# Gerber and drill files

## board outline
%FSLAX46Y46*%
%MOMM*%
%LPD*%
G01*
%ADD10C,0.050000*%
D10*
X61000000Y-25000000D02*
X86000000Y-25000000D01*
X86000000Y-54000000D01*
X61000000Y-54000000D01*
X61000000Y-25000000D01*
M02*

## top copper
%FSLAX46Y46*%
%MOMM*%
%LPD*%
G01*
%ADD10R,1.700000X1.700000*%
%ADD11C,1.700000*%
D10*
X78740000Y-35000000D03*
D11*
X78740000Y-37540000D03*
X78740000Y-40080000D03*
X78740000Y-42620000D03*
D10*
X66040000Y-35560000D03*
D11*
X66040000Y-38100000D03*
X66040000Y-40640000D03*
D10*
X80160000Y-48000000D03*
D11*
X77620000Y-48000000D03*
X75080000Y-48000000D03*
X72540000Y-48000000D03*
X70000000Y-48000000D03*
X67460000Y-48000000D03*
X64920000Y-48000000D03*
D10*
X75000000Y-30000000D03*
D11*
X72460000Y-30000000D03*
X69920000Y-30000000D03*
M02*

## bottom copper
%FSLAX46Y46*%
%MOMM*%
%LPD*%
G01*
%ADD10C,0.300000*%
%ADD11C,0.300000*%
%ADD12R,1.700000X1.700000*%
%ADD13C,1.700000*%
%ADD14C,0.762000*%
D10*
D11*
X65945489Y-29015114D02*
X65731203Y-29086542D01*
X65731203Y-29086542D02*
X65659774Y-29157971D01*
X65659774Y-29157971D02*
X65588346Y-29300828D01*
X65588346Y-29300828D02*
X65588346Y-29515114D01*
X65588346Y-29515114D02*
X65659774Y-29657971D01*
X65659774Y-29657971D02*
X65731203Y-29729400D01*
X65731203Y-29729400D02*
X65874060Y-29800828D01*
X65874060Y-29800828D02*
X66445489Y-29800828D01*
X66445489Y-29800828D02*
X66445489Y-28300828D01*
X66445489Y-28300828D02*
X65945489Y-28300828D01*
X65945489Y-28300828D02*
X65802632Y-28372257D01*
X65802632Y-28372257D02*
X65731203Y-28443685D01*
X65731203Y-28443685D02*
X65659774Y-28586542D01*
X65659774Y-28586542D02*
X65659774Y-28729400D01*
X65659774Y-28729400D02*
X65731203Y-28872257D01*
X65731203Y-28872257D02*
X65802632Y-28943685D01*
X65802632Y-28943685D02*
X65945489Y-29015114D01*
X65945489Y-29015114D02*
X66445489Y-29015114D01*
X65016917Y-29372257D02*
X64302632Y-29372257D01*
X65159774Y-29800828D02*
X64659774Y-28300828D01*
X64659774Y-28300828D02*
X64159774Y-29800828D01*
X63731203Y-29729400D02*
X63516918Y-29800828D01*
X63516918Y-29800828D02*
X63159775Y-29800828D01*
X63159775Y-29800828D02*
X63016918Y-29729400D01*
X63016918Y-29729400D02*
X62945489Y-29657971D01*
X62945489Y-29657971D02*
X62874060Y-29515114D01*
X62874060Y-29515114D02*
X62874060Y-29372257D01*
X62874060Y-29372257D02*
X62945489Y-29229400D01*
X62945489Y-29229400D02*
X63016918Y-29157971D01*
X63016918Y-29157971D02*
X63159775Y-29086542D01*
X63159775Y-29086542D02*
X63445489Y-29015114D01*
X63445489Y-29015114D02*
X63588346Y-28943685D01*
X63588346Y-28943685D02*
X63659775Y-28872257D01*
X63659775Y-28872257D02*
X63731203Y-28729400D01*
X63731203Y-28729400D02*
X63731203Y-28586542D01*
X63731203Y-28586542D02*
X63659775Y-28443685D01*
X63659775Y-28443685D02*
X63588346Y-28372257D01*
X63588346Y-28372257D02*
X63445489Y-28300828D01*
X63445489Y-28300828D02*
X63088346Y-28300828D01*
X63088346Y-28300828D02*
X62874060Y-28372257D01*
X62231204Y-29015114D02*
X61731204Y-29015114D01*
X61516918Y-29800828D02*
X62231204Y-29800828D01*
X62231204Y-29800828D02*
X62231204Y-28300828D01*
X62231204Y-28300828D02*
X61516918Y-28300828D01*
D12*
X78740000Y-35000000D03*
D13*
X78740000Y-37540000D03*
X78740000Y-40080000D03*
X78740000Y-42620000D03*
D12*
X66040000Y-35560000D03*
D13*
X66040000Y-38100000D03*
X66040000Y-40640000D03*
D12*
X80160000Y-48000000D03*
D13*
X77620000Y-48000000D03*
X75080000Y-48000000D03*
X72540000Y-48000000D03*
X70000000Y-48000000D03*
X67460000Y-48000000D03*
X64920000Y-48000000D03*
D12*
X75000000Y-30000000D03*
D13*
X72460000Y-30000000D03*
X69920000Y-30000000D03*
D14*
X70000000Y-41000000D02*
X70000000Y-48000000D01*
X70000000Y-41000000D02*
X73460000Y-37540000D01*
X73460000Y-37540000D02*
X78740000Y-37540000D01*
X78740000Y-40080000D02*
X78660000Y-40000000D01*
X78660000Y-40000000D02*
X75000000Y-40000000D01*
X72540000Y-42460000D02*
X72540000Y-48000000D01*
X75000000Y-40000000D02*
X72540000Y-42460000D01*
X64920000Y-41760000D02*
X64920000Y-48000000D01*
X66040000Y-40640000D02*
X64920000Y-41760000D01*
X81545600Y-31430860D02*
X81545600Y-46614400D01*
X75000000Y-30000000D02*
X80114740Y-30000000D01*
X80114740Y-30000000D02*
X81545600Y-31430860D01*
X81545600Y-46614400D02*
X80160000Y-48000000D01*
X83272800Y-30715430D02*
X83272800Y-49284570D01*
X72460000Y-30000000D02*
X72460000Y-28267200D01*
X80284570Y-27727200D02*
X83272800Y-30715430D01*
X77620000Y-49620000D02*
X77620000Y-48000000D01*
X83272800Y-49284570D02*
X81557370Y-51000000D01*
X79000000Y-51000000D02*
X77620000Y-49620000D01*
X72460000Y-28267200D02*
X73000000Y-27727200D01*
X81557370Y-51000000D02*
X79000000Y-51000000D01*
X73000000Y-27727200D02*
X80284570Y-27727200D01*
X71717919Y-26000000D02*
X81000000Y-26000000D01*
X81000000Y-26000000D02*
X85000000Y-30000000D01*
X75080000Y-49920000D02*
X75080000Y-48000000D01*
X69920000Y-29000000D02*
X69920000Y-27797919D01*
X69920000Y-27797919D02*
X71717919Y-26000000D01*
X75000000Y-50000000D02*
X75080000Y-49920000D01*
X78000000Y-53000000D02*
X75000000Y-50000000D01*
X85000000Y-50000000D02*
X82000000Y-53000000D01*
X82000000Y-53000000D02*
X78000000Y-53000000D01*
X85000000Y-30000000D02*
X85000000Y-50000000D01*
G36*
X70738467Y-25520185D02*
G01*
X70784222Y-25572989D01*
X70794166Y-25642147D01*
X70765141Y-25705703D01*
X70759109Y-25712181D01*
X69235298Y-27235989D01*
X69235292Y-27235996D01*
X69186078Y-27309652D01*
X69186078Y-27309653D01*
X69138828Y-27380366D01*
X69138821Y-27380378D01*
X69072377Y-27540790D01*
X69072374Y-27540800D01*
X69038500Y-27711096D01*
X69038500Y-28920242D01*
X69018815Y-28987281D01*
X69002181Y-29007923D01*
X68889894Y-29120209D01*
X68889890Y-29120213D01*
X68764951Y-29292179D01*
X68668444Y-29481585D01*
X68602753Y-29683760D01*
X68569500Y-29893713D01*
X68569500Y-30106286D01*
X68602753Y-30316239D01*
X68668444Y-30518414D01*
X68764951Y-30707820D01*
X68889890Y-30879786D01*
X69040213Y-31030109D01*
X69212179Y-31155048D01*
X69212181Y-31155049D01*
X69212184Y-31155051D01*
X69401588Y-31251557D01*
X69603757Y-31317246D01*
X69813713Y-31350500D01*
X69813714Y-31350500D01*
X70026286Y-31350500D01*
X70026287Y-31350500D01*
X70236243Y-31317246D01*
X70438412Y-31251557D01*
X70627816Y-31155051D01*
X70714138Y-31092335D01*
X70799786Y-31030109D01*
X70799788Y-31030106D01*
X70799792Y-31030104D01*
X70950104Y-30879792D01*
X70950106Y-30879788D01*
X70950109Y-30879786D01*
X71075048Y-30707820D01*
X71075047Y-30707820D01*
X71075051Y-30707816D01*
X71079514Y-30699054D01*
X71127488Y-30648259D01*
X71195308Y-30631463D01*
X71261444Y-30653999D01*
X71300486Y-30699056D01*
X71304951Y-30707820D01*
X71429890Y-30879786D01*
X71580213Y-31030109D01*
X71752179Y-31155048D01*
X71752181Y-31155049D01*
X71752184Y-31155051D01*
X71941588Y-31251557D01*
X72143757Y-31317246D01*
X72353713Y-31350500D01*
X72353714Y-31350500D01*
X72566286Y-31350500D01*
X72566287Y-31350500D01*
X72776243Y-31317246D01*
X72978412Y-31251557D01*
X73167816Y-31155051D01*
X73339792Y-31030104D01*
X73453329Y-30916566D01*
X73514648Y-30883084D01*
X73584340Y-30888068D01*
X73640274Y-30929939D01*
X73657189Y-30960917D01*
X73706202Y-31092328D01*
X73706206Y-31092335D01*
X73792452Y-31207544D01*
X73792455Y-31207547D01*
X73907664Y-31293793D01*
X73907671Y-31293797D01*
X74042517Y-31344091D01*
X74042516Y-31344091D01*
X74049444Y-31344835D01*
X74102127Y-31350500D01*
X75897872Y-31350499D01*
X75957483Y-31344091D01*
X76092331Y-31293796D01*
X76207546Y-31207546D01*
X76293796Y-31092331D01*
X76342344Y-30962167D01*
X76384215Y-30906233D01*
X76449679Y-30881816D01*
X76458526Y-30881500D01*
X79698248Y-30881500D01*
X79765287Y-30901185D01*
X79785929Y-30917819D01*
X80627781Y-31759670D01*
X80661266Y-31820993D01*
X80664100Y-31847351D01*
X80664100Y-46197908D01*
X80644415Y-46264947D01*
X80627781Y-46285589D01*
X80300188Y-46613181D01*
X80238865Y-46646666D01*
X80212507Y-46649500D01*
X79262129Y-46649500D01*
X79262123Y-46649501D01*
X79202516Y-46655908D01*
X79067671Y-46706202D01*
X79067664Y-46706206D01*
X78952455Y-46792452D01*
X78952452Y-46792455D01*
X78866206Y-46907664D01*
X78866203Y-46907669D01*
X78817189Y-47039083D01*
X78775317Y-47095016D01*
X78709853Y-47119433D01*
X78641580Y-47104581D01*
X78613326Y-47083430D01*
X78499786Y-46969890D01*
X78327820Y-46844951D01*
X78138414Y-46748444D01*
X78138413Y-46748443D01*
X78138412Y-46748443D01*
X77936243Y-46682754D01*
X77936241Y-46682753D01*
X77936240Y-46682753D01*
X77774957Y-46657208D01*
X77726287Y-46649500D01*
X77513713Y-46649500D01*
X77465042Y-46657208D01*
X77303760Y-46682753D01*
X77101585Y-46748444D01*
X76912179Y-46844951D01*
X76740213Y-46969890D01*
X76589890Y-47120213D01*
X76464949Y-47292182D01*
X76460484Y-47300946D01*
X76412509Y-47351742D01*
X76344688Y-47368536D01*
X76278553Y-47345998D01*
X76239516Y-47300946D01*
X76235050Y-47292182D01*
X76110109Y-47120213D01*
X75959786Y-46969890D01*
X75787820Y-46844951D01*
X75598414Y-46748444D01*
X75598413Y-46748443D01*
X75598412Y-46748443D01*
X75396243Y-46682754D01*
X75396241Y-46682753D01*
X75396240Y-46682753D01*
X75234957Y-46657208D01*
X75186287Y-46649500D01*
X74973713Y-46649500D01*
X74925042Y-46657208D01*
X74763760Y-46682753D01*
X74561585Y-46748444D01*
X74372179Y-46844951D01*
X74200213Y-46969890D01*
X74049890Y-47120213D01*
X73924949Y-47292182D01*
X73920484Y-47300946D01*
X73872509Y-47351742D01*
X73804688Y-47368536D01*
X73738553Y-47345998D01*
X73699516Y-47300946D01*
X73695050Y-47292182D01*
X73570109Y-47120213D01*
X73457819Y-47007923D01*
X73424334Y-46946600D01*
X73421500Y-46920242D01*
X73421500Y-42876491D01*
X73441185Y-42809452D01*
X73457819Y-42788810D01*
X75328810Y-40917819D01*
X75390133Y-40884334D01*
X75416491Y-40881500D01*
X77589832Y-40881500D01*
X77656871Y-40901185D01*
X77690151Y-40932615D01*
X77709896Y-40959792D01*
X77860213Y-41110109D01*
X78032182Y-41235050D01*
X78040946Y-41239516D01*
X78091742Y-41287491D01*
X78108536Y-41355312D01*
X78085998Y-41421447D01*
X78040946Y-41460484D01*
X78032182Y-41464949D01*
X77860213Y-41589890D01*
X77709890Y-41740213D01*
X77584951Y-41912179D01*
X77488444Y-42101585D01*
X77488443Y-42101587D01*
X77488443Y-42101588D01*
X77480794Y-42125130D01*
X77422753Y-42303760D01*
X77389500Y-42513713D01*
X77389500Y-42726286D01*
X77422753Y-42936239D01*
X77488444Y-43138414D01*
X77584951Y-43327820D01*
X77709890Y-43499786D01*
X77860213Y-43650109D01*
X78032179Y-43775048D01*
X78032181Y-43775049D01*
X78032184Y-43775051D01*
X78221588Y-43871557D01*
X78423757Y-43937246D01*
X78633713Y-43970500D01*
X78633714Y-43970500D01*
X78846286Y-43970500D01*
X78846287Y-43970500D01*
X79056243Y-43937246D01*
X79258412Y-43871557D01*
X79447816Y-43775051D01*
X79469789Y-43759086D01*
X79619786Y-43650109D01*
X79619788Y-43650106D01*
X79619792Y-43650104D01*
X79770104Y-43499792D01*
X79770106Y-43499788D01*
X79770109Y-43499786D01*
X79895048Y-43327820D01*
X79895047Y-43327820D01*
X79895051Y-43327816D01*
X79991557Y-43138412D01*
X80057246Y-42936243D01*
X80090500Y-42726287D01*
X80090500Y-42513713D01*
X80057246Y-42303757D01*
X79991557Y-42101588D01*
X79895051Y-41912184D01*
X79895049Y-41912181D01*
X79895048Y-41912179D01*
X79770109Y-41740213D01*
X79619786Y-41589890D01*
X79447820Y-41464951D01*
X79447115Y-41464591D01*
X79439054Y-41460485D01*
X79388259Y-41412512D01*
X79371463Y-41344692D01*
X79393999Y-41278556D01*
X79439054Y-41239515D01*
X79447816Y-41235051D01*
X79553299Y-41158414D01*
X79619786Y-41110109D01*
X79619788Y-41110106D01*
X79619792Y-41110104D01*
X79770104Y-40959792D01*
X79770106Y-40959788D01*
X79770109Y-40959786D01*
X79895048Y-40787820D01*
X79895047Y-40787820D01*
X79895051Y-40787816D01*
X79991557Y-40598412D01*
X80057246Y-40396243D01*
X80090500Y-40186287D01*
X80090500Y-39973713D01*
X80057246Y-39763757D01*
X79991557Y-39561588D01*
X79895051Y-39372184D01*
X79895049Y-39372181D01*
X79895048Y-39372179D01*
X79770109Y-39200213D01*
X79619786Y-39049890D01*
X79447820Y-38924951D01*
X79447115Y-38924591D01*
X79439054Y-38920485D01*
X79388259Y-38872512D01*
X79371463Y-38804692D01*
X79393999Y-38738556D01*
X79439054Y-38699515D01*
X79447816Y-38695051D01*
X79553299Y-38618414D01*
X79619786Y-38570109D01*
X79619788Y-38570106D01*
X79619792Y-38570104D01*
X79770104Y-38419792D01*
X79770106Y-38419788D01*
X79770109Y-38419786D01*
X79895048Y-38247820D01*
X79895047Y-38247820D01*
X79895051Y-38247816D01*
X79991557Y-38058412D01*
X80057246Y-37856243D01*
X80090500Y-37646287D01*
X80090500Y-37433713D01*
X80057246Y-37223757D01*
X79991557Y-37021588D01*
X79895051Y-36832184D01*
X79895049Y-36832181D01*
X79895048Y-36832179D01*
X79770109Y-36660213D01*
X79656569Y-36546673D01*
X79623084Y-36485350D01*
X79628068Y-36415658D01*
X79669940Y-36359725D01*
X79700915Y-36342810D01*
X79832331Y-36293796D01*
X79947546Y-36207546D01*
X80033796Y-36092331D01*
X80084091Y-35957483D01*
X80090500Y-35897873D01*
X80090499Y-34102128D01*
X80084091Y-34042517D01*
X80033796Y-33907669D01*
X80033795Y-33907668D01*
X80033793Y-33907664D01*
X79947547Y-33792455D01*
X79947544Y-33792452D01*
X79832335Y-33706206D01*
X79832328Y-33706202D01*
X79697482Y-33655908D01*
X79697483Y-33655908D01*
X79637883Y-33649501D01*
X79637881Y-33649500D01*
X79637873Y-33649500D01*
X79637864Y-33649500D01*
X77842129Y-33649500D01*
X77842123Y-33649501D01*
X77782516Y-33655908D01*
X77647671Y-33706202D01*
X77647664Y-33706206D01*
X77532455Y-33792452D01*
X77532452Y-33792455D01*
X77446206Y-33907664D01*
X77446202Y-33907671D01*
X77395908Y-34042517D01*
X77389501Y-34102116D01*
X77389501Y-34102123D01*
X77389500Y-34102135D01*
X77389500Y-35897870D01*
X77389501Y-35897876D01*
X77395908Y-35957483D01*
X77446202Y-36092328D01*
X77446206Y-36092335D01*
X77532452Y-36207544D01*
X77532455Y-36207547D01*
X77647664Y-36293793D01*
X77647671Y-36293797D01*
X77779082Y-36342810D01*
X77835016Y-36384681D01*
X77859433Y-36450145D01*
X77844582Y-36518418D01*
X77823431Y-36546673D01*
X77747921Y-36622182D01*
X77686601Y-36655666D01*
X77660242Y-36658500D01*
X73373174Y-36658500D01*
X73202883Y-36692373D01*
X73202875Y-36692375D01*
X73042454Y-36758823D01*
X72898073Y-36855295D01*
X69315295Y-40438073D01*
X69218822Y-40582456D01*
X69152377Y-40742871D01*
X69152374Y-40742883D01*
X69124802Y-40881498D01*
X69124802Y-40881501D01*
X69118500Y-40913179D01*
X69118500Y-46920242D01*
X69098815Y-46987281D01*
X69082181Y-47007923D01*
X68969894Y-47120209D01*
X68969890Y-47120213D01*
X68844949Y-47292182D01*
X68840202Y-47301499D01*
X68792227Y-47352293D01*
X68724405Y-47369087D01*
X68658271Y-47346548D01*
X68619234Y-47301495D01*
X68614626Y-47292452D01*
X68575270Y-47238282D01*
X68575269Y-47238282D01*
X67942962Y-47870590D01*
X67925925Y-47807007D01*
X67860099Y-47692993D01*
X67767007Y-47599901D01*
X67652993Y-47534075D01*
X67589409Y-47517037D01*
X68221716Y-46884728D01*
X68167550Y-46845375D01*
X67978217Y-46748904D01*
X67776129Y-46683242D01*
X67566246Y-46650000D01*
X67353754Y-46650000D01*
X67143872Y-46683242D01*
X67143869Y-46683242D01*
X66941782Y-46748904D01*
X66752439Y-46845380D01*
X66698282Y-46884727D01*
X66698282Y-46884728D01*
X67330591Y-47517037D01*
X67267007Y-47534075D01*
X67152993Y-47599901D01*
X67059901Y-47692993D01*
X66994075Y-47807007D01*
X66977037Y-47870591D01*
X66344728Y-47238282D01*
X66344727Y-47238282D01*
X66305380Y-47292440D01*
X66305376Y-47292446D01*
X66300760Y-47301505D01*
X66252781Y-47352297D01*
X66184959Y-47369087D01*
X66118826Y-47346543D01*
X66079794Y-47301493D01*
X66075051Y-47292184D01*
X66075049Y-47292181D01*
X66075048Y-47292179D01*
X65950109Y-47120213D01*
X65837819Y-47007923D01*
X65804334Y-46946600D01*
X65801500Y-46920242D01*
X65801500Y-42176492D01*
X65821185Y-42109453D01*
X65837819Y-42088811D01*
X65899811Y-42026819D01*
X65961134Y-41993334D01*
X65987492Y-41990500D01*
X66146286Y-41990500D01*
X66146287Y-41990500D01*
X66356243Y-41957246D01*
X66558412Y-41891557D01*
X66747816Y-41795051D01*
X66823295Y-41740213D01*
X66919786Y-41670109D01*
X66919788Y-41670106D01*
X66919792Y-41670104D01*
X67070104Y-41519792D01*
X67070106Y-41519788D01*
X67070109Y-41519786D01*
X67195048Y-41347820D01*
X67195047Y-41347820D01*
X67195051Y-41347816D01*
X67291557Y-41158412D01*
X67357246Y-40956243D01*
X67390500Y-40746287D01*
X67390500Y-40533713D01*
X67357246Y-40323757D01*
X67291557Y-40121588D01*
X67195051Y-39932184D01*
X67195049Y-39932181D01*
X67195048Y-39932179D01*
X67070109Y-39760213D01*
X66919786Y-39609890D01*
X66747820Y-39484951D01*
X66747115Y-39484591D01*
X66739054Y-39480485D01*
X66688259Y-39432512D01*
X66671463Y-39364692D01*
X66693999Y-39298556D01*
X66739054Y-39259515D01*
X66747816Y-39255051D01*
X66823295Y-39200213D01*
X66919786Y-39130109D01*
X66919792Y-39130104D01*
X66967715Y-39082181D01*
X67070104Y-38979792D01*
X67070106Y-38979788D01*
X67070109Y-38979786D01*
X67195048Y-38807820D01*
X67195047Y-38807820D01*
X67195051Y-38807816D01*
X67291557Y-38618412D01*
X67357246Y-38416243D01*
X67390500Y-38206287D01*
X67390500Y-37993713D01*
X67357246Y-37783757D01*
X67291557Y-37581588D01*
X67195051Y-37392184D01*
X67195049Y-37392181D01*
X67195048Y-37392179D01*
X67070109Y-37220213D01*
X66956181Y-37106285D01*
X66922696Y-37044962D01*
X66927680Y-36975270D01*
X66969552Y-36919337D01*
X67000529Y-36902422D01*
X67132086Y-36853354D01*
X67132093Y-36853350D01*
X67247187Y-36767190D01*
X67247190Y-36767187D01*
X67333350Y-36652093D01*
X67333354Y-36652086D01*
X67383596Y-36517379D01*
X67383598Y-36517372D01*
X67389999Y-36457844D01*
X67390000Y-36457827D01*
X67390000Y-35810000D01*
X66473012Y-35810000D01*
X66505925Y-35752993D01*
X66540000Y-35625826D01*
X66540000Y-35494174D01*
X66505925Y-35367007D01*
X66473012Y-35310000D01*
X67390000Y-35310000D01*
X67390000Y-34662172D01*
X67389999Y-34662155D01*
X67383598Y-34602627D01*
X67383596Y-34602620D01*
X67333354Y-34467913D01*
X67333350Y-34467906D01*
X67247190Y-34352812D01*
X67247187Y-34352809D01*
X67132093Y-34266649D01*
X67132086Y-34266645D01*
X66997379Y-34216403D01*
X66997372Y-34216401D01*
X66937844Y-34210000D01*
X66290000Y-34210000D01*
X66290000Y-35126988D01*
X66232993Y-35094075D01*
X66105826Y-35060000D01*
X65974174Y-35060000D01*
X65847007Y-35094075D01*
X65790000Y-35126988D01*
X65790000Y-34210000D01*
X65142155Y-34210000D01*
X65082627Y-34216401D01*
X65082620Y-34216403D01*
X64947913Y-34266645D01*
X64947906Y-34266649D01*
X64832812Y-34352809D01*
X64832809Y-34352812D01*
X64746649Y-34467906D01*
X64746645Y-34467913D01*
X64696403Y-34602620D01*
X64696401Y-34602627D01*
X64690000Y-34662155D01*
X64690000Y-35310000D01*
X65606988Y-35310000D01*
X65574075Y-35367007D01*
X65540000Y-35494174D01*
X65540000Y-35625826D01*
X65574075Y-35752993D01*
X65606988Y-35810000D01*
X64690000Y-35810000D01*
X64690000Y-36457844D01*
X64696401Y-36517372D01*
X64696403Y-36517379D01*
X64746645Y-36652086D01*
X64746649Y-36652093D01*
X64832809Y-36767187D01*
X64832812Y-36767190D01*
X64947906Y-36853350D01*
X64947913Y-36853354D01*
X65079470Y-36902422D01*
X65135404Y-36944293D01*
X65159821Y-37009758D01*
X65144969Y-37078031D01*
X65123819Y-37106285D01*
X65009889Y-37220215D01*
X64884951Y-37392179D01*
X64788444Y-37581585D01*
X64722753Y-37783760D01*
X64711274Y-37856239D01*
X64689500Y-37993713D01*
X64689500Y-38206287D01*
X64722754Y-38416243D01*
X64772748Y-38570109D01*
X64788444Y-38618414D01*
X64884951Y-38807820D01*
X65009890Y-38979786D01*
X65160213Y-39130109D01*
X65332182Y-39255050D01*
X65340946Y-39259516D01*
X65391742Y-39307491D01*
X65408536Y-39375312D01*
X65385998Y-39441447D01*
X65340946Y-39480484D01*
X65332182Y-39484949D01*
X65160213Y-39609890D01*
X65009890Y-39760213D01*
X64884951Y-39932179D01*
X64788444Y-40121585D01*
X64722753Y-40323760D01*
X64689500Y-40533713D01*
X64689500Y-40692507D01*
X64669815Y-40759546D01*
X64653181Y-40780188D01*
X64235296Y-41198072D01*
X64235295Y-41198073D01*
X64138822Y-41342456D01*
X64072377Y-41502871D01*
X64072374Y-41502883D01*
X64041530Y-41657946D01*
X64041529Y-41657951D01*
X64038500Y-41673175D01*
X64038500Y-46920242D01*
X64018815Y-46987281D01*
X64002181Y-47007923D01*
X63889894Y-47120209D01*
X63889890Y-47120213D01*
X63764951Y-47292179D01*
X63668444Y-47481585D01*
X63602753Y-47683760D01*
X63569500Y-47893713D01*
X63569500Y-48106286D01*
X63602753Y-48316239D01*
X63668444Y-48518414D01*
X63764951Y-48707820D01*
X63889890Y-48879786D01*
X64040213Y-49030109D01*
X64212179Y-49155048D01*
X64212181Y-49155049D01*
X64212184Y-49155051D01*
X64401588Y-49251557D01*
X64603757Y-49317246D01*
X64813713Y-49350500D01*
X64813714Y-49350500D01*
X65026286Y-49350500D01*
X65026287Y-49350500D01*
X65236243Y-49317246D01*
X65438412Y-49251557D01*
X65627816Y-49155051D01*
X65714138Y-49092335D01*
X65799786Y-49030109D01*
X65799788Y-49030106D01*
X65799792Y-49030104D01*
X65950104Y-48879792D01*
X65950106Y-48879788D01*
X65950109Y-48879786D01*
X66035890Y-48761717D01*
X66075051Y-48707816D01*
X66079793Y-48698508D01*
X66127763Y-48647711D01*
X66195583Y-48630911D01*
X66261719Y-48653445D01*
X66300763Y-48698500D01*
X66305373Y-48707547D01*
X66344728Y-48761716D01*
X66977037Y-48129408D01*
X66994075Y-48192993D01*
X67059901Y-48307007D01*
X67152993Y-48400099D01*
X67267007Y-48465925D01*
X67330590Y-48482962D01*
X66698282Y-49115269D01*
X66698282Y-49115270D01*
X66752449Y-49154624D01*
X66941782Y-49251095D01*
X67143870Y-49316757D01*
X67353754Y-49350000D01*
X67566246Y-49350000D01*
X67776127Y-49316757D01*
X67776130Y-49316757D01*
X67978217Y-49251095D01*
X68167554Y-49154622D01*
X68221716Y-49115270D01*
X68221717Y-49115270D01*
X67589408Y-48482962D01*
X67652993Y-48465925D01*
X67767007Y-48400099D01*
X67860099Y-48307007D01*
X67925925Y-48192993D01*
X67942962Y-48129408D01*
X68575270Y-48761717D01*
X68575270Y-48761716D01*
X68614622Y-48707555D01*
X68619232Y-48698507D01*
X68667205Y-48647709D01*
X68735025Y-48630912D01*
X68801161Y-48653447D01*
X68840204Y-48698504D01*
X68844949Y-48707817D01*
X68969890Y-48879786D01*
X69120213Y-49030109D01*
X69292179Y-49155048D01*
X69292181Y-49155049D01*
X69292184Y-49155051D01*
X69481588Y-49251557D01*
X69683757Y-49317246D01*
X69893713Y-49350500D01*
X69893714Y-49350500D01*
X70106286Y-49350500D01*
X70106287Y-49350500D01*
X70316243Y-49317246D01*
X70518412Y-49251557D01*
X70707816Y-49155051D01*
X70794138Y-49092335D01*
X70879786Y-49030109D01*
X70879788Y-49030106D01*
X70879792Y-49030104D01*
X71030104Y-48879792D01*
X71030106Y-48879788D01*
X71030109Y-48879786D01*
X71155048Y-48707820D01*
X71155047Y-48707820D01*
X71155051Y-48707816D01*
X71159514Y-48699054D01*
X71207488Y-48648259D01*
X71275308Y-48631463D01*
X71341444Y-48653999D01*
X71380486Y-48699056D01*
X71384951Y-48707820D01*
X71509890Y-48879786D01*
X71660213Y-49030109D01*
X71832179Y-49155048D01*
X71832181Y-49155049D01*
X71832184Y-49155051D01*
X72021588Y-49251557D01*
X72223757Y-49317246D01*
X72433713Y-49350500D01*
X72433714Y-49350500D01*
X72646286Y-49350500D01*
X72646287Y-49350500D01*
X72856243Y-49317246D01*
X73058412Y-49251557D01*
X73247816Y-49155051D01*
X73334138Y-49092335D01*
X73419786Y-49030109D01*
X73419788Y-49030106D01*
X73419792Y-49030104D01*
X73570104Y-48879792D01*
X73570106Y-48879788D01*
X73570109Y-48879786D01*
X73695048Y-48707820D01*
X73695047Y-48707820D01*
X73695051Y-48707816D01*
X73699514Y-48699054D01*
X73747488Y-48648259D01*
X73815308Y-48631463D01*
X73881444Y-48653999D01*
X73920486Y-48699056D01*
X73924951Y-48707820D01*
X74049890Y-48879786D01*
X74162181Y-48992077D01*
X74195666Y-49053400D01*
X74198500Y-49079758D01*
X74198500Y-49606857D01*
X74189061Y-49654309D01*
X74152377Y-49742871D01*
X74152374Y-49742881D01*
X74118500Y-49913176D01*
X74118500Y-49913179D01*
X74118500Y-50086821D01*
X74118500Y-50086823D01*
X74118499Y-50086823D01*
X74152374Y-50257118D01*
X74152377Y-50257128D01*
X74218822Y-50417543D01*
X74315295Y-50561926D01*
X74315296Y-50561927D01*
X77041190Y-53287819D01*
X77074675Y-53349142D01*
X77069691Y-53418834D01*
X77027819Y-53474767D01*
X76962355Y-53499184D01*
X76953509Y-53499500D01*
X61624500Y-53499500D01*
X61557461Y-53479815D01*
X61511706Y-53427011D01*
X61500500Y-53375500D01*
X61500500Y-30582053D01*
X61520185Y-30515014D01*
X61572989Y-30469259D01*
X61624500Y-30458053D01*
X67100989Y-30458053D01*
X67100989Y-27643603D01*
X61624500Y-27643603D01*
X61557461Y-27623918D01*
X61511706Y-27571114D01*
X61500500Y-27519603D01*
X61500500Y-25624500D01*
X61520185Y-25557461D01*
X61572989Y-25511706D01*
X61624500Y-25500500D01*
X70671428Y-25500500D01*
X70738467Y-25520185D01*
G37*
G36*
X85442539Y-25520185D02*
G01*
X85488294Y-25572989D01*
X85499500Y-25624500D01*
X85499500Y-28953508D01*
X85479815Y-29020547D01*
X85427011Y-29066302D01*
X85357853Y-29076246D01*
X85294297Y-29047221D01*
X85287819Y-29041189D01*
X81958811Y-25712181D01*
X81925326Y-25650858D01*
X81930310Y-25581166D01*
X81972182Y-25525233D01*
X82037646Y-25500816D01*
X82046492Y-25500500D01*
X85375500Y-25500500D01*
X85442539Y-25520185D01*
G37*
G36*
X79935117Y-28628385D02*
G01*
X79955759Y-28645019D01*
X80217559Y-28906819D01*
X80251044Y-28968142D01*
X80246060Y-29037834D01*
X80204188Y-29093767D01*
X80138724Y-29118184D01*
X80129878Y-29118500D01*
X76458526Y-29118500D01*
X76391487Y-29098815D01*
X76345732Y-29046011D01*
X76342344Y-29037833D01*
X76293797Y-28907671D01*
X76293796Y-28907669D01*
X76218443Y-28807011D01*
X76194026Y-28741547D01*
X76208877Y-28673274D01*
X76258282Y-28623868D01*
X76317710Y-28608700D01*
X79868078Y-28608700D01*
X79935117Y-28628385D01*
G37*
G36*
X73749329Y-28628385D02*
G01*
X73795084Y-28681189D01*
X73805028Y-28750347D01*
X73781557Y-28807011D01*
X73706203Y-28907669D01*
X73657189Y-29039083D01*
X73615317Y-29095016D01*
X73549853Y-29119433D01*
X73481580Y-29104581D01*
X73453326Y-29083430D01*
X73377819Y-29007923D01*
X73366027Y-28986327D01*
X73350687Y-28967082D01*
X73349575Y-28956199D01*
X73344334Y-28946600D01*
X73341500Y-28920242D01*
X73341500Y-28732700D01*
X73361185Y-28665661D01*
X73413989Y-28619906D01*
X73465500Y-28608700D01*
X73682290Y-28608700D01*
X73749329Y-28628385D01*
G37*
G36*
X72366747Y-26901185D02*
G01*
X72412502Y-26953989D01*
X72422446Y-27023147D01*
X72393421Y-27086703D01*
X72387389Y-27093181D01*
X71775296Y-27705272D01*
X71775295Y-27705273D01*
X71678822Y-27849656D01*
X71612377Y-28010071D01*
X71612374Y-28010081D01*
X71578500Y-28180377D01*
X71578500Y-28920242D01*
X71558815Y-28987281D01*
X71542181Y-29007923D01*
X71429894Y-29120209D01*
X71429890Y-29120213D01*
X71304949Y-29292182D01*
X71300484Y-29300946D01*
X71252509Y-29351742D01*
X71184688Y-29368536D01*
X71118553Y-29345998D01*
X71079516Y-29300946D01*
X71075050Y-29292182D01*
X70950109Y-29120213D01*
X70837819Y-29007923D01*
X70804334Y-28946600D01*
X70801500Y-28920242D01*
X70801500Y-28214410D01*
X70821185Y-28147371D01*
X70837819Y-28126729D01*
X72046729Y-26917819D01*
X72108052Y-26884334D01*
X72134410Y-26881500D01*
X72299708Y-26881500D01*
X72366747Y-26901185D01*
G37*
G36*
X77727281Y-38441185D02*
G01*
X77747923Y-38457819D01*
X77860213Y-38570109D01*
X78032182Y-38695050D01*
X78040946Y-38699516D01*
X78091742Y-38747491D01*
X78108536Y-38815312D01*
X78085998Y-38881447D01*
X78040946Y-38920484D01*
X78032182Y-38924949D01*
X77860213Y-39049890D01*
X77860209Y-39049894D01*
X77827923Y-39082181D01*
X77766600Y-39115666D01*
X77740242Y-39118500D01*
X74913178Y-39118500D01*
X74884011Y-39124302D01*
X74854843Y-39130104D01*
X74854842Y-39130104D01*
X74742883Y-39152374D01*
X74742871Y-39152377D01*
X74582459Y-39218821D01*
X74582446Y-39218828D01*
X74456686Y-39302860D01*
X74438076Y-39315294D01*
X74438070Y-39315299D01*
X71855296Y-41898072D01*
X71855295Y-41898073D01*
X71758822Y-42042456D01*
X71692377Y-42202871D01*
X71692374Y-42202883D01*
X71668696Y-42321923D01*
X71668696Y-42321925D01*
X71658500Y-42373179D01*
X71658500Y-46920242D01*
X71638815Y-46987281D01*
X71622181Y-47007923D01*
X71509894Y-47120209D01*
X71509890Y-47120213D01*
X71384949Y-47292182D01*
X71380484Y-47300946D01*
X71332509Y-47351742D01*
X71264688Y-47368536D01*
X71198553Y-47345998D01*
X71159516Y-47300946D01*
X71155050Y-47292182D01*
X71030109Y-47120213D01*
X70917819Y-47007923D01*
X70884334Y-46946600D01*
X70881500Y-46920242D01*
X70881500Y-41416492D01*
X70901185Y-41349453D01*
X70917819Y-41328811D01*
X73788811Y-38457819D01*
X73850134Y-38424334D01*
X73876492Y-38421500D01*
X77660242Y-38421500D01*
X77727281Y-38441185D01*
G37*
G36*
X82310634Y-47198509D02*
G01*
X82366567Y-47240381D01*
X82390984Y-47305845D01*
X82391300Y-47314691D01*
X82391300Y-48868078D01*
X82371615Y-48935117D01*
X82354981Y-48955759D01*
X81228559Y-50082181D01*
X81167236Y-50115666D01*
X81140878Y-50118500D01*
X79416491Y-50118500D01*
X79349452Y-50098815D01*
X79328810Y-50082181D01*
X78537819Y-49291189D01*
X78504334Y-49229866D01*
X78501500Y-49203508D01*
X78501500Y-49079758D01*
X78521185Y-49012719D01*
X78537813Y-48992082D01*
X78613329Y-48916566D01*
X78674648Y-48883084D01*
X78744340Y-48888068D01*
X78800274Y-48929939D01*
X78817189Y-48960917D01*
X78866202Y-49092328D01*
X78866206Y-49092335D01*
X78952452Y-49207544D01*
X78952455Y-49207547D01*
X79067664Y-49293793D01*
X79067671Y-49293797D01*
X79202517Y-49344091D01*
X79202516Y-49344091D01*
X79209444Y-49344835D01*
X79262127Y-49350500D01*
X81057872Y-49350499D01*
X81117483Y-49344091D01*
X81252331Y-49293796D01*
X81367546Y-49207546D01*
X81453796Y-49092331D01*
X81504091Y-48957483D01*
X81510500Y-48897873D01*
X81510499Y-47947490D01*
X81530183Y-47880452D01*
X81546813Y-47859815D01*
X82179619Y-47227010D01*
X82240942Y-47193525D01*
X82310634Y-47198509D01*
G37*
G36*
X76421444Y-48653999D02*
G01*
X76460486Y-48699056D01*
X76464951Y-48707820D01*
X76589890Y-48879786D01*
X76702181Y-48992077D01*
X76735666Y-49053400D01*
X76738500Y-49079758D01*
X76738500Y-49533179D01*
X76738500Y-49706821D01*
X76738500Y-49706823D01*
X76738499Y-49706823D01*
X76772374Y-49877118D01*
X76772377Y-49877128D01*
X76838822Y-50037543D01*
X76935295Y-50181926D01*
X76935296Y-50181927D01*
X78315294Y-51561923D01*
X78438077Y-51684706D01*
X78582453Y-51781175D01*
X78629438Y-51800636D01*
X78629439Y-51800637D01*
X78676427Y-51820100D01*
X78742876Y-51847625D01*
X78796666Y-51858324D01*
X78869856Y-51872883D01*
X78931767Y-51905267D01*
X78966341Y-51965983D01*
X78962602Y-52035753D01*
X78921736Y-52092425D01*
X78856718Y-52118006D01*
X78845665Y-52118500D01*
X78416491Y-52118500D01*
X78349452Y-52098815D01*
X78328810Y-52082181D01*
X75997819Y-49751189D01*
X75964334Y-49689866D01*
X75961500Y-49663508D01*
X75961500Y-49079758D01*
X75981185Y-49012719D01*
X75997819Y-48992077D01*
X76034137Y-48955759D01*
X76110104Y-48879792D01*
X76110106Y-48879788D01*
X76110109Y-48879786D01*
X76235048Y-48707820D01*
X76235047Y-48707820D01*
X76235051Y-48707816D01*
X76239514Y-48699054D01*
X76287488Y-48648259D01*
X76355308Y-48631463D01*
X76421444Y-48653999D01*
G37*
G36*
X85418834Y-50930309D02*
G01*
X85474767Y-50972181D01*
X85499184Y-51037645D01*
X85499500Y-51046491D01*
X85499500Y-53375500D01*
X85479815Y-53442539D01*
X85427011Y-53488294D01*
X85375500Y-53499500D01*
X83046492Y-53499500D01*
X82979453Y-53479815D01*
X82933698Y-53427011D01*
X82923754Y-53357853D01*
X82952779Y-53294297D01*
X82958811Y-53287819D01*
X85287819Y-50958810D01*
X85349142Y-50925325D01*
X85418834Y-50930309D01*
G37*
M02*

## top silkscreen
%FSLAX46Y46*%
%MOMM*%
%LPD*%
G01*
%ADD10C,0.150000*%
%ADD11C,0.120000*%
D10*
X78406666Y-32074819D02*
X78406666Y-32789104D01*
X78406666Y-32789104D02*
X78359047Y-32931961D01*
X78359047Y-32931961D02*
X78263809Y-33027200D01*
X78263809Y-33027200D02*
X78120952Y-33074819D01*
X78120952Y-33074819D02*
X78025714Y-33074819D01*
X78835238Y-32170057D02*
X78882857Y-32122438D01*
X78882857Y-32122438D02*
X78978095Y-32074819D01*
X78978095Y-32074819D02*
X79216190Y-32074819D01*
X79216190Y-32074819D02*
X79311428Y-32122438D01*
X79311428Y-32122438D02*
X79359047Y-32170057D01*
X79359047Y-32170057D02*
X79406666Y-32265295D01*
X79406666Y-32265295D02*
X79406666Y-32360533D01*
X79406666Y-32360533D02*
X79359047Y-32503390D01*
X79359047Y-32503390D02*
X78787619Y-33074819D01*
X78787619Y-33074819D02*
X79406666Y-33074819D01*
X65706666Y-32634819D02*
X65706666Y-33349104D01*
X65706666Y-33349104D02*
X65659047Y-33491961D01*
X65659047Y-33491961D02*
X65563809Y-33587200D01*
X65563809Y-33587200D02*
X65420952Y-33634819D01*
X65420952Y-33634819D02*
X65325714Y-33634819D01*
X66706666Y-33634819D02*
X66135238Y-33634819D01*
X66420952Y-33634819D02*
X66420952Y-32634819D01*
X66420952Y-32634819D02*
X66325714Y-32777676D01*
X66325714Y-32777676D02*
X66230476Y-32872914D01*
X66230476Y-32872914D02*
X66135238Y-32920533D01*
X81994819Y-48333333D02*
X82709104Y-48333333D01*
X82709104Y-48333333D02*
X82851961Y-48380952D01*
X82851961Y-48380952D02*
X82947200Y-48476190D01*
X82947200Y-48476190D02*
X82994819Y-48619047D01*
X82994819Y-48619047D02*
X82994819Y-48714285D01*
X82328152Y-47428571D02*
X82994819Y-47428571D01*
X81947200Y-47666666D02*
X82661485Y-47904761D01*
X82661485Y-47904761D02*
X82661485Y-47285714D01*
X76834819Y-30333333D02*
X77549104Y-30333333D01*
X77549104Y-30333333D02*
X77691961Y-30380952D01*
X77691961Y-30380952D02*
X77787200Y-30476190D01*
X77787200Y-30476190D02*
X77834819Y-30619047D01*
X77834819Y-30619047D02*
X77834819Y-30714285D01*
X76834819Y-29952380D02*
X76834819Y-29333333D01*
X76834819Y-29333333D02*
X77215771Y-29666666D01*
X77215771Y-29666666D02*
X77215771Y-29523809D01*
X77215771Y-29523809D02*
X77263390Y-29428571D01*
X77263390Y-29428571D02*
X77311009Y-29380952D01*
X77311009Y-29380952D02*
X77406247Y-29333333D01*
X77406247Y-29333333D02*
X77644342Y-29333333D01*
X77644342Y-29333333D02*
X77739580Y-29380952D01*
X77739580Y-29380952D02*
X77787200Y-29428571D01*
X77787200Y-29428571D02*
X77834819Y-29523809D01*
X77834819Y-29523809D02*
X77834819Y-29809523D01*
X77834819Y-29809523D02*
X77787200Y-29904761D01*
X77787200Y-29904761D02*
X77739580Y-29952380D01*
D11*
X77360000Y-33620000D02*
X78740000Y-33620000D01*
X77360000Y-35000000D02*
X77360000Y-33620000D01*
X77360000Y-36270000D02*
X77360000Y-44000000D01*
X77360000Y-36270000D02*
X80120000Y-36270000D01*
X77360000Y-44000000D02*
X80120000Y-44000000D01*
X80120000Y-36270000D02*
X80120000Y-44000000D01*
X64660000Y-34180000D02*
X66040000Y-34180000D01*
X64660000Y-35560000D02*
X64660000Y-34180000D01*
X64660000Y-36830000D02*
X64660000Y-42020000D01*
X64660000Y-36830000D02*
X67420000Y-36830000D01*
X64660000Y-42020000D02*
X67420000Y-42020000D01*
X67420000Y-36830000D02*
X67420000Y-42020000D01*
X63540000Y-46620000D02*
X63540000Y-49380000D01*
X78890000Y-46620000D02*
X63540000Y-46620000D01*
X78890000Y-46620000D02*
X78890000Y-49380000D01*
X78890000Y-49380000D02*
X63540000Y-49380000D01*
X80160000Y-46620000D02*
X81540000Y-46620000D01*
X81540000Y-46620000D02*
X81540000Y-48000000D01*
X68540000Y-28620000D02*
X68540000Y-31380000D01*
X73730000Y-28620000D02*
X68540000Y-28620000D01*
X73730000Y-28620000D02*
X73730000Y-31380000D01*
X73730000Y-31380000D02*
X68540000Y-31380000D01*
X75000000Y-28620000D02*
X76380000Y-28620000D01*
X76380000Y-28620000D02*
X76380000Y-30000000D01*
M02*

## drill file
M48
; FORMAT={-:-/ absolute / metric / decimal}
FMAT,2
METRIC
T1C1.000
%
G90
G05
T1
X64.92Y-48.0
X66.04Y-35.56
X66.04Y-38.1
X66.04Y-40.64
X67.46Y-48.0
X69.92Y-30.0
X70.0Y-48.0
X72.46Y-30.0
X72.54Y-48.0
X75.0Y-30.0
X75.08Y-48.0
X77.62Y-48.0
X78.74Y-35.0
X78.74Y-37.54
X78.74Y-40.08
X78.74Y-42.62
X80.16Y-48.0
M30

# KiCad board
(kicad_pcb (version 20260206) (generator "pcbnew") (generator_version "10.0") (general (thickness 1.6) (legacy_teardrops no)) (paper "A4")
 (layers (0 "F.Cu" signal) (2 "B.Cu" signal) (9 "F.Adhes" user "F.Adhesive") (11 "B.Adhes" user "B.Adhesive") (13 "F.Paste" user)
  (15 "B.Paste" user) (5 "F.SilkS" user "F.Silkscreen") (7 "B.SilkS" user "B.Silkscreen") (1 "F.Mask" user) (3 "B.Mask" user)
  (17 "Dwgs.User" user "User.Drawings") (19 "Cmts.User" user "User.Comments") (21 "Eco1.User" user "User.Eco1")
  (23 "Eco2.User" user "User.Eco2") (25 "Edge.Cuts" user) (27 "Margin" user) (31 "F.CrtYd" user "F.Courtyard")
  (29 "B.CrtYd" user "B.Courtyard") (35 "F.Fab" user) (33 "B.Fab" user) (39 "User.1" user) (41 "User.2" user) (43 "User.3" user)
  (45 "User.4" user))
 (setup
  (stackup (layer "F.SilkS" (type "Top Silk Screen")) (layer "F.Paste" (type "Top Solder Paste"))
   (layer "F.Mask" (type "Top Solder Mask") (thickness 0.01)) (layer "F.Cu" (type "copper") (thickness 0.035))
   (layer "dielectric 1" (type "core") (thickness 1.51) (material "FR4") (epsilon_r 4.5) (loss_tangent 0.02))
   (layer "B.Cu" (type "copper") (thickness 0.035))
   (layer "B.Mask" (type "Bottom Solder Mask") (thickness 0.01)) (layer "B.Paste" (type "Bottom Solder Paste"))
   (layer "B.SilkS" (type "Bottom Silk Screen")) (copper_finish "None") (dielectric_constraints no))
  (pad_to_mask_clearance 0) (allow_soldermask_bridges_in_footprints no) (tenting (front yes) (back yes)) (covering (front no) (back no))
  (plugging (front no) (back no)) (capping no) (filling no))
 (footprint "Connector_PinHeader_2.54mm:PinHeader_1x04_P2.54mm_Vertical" (layer "F.Cu") (at 78.74 35)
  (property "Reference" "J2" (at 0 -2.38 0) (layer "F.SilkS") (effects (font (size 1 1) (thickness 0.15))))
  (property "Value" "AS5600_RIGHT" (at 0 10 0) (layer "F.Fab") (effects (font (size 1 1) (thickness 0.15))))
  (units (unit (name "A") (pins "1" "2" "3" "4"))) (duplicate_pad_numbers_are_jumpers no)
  (fp_line (start -1.38 -1.38) (end 0 -1.38) (stroke (width 0.12) (type solid)) (layer "F.SilkS"))
  (fp_line (start -1.38 0) (end -1.38 -1.38) (stroke (width 0.12) (type solid)) (layer "F.SilkS"))
  (fp_line (start -1.38 1.27) (end -1.38 9) (stroke (width 0.12) (type solid)) (layer "F.SilkS"))
  (fp_line (start -1.38 1.27) (end 1.38 1.27) (stroke (width 0.12) (type solid)) (layer "F.SilkS"))
  (fp_line (start -1.38 9) (end 1.38 9) (stroke (width 0.12) (type solid)) (layer "F.SilkS"))
  (fp_line (start 1.38 1.27) (end 1.38 9) (stroke (width 0.12) (type solid)) (layer "F.SilkS"))
  (pad "1" thru_hole rect (at 0 0) (size 1.7 1.7) (drill 1) (layers "*.Cu" "*.Mask") (remove_unused_layers no)
   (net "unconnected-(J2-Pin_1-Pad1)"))
  (pad "2" thru_hole circle (at 0 2.54) (size 1.7 1.7) (drill 1) (layers "*.Cu" "*.Mask") (remove_unused_layers no) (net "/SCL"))
  (pad "3" thru_hole circle (at 0 5.08) (size 1.7 1.7) (drill 1) (layers "*.Cu" "*.Mask") (remove_unused_layers no) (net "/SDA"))
  (pad "4" thru_hole circle (at 0 7.62) (size 1.7 1.7) (drill 1) (layers "*.Cu" "*.Mask") (remove_unused_layers no)
   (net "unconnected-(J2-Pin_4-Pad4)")))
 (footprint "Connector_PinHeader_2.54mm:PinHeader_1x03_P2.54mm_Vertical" (layer "F.Cu") (at 66.04 35.56)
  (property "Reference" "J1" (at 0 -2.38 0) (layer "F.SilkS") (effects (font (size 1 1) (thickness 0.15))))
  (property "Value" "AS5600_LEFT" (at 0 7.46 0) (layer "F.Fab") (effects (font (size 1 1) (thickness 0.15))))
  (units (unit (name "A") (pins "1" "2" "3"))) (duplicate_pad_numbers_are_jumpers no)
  (fp_line (start -1.38 -1.38) (end 0 -1.38) (stroke (width 0.12) (type solid)) (layer "F.SilkS"))
  (fp_line (start -1.38 0) (end -1.38 -1.38) (stroke (width 0.12) (type solid)) (layer "F.SilkS"))
  (fp_line (start -1.38 1.27) (end -1.38 6.46) (stroke (width 0.12) (type solid)) (layer "F.SilkS"))
  (fp_line (start -1.38 1.27) (end 1.38 1.27) (stroke (width 0.12) (type solid)) (layer "F.SilkS"))
  (fp_line (start -1.38 6.46) (end 1.38 6.46) (stroke (width 0.12) (type solid)) (layer "F.SilkS"))
  (fp_line (start 1.38 1.27) (end 1.38 6.46) (stroke (width 0.12) (type solid)) (layer "F.SilkS"))
  (pad "1" thru_hole rect (at 0 0) (size 1.7 1.7) (drill 1) (layers "*.Cu" "*.Mask") (remove_unused_layers no) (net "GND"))
  (pad "2" thru_hole circle (at 0 2.54) (size 1.7 1.7) (drill 1) (layers "*.Cu" "*.Mask") (remove_unused_layers no)
   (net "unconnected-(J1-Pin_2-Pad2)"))
  (pad "3" thru_hole circle (at 0 5.08) (size 1.7 1.7) (drill 1) (layers "*.Cu" "*.Mask") (remove_unused_layers no) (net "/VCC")))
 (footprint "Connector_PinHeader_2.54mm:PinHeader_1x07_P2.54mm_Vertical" (layer "F.Cu") (at 80.16 48 -90)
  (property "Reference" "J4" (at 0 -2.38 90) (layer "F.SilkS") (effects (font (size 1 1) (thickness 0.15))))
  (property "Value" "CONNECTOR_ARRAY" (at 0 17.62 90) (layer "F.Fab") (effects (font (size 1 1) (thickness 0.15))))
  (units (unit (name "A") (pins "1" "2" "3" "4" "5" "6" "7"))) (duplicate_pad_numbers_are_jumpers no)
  (fp_line (start -1.38 16.62) (end 1.38 16.62) (stroke (width 0.12) (type solid)) (layer "F.SilkS"))
  (fp_line (start -1.38 1.27) (end -1.38 16.62) (stroke (width 0.12) (type solid)) (layer "F.SilkS"))
  (fp_line (start -1.38 1.27) (end 1.38 1.27) (stroke (width 0.12) (type solid)) (layer "F.SilkS"))
  (fp_line (start 1.38 1.27) (end 1.38 16.62) (stroke (width 0.12) (type solid)) (layer "F.SilkS"))
  (fp_line (start -1.38 0) (end -1.38 -1.38) (stroke (width 0.12) (type solid)) (layer "F.SilkS"))
  (fp_line (start -1.38 -1.38) (end 0 -1.38) (stroke (width 0.12) (type solid)) (layer "F.SilkS"))
  (pad "1" thru_hole rect (at 0 0 270) (size 1.7 1.7) (drill 1) (layers "*.Cu" "*.Mask") (remove_unused_layers no) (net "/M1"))
  (pad "2" thru_hole circle (at 0 2.54 270) (size 1.7 1.7) (drill 1) (layers "*.Cu" "*.Mask") (remove_unused_layers no) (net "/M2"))
  (pad "3" thru_hole circle (at 0 5.08 270) (size 1.7 1.7) (drill 1) (layers "*.Cu" "*.Mask") (remove_unused_layers no) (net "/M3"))
  (pad "4" thru_hole circle (at 0 7.62 270) (size 1.7 1.7) (drill 1) (layers "*.Cu" "*.Mask") (remove_unused_layers no) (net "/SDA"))
  (pad "5" thru_hole circle (at 0 10.16 270) (size 1.7 1.7) (drill 1) (layers "*.Cu" "*.Mask") (remove_unused_layers no) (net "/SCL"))
  (pad "6" thru_hole circle (at 0 12.7 270) (size 1.7 1.7) (drill 1) (layers "*.Cu" "*.Mask") (remove_unused_layers no) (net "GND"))
  (pad "7" thru_hole circle (at 0 15.24 270) (size 1.7 1.7) (drill 1) (layers "*.Cu" "*.Mask") (remove_unused_layers no) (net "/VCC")))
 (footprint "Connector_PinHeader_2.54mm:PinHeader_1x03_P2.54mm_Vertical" (layer "F.Cu") (at 75 30 -90)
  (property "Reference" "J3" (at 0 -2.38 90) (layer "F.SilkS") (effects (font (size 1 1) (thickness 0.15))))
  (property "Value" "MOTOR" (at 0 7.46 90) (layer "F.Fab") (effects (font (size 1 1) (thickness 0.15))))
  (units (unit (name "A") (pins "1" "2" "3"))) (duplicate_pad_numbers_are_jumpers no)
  (fp_line (start -1.38 6.46) (end 1.38 6.46) (stroke (width 0.12) (type solid)) (layer "F.SilkS"))
  (fp_line (start -1.38 1.27) (end -1.38 6.46) (stroke (width 0.12) (type solid)) (layer "F.SilkS"))
  (fp_line (start -1.38 1.27) (end 1.38 1.27) (stroke (width 0.12) (type solid)) (layer "F.SilkS"))
  (fp_line (start 1.38 1.27) (end 1.38 6.46) (stroke (width 0.12) (type solid)) (layer "F.SilkS"))
  (fp_line (start -1.38 0) (end -1.38 -1.38) (stroke (width 0.12) (type solid)) (layer "F.SilkS"))
  (fp_line (start -1.38 -1.38) (end 0 -1.38) (stroke (width 0.12) (type solid)) (layer "F.SilkS"))
  (pad "1" thru_hole rect (at 0 0 270) (size 1.7 1.7) (drill 1) (layers "*.Cu" "*.Mask") (remove_unused_layers no) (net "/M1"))
  (pad "2" thru_hole circle (at 0 2.54 270) (size 1.7 1.7) (drill 1) (layers "*.Cu" "*.Mask") (remove_unused_layers no) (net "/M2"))
  (pad "3" thru_hole circle (at 0 5.08 270) (size 1.7 1.7) (drill 1) (layers "*.Cu" "*.Mask") (remove_unused_layers no) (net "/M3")))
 (gr_rect (start 61 25) (end 86 54) (stroke (width 0.05) (type default)) (fill no) (layer "Edge.Cuts"))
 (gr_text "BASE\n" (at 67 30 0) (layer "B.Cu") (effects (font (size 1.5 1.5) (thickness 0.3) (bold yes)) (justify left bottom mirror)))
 (segment (start 70 41) (end 70 48) (width 0.762) (layer "B.Cu") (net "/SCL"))
 (segment (start 70 41) (end 73.46 37.54) (width 0.762) (layer "B.Cu") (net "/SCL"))
 (segment (start 73.46 37.54) (end 78.74 37.54) (width 0.762) (layer "B.Cu") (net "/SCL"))
 (segment (start 78.74 40.08) (end 78.66 40) (width 0.762) (layer "B.Cu") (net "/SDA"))
 (segment (start 78.66 40) (end 75 40) (width 0.762) (layer "B.Cu") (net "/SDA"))
 (segment (start 72.54 42.46) (end 72.54 48) (width 0.762) (layer "B.Cu") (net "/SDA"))
 (segment (start 75 40) (end 72.54 42.46) (width 0.762) (layer "B.Cu") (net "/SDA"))
 (segment (start 64.92 41.76) (end 64.92 48) (width 0.762) (layer "B.Cu") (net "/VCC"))
 (segment (start 66.04 40.64) (end 64.92 41.76) (width 0.762) (layer "B.Cu") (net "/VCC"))
 (segment (start 81.5456 31.43086) (end 81.5456 46.6144) (width 0.762) (layer "B.Cu") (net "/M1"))
 (segment (start 75 30) (end 80.11474 30) (width 0.762) (layer "B.Cu") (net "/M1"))
 (segment (start 80.11474 30) (end 81.5456 31.43086) (width 0.762) (layer "B.Cu") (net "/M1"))
 (segment (start 81.5456 46.6144) (end 80.16 48) (width 0.762) (layer "B.Cu") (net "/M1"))
 (segment (start 83.2728 30.71543) (end 83.2728 49.28457) (width 0.762) (layer "B.Cu") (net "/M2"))
 (segment (start 72.46 30) (end 72.46 28.2672) (width 0.762) (layer "B.Cu") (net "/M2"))
 (segment (start 80.28457 27.7272) (end 83.2728 30.71543) (width 0.762) (layer "B.Cu") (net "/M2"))
 (segment (start 77.62 49.62) (end 77.62 48) (width 0.762) (layer "B.Cu") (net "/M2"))
 (segment (start 83.2728 49.28457) (end 81.55737 51) (width 0.762) (layer "B.Cu") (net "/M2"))
 (segment (start 79 51) (end 77.62 49.62) (width 0.762) (layer "B.Cu") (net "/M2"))
 (segment (start 72.46 28.2672) (end 73 27.7272) (width 0.762) (layer "B.Cu") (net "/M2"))
 (segment (start 81.55737 51) (end 79 51) (width 0.762) (layer "B.Cu") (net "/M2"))
 (segment (start 73 27.7272) (end 80.28457 27.7272) (width 0.762) (layer "B.Cu") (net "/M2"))
 (segment (start 71.717919 26) (end 81 26) (width 0.762) (layer "B.Cu") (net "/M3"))
 (segment (start 81 26) (end 85 30) (width 0.762) (layer "B.Cu") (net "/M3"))
 (segment (start 75.08 49.92) (end 75.08 48) (width 0.762) (layer "B.Cu") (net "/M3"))
 (segment (start 69.92 29) (end 69.92 27.797919) (width 0.762) (layer "B.Cu") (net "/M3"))
 (segment (start 69.92 27.797919) (end 71.717919 26) (width 0.762) (layer "B.Cu") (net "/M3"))
 (segment (start 75 50) (end 75.08 49.92) (width 0.762) (layer "B.Cu") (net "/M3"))
 (segment (start 78 53) (end 75 50) (width 0.762) (layer "B.Cu") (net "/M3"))
 (segment (start 85 50) (end 82 53) (width 0.762) (layer "B.Cu") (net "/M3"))
 (segment (start 82 53) (end 78 53) (width 0.762) (layer "B.Cu") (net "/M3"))
 (segment (start 85 30) (end 85 50) (width 0.762) (layer "B.Cu") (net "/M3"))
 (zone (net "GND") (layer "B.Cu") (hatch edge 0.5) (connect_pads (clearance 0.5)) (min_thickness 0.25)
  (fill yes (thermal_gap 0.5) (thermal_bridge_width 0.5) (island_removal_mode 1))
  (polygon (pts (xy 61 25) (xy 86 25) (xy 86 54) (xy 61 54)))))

